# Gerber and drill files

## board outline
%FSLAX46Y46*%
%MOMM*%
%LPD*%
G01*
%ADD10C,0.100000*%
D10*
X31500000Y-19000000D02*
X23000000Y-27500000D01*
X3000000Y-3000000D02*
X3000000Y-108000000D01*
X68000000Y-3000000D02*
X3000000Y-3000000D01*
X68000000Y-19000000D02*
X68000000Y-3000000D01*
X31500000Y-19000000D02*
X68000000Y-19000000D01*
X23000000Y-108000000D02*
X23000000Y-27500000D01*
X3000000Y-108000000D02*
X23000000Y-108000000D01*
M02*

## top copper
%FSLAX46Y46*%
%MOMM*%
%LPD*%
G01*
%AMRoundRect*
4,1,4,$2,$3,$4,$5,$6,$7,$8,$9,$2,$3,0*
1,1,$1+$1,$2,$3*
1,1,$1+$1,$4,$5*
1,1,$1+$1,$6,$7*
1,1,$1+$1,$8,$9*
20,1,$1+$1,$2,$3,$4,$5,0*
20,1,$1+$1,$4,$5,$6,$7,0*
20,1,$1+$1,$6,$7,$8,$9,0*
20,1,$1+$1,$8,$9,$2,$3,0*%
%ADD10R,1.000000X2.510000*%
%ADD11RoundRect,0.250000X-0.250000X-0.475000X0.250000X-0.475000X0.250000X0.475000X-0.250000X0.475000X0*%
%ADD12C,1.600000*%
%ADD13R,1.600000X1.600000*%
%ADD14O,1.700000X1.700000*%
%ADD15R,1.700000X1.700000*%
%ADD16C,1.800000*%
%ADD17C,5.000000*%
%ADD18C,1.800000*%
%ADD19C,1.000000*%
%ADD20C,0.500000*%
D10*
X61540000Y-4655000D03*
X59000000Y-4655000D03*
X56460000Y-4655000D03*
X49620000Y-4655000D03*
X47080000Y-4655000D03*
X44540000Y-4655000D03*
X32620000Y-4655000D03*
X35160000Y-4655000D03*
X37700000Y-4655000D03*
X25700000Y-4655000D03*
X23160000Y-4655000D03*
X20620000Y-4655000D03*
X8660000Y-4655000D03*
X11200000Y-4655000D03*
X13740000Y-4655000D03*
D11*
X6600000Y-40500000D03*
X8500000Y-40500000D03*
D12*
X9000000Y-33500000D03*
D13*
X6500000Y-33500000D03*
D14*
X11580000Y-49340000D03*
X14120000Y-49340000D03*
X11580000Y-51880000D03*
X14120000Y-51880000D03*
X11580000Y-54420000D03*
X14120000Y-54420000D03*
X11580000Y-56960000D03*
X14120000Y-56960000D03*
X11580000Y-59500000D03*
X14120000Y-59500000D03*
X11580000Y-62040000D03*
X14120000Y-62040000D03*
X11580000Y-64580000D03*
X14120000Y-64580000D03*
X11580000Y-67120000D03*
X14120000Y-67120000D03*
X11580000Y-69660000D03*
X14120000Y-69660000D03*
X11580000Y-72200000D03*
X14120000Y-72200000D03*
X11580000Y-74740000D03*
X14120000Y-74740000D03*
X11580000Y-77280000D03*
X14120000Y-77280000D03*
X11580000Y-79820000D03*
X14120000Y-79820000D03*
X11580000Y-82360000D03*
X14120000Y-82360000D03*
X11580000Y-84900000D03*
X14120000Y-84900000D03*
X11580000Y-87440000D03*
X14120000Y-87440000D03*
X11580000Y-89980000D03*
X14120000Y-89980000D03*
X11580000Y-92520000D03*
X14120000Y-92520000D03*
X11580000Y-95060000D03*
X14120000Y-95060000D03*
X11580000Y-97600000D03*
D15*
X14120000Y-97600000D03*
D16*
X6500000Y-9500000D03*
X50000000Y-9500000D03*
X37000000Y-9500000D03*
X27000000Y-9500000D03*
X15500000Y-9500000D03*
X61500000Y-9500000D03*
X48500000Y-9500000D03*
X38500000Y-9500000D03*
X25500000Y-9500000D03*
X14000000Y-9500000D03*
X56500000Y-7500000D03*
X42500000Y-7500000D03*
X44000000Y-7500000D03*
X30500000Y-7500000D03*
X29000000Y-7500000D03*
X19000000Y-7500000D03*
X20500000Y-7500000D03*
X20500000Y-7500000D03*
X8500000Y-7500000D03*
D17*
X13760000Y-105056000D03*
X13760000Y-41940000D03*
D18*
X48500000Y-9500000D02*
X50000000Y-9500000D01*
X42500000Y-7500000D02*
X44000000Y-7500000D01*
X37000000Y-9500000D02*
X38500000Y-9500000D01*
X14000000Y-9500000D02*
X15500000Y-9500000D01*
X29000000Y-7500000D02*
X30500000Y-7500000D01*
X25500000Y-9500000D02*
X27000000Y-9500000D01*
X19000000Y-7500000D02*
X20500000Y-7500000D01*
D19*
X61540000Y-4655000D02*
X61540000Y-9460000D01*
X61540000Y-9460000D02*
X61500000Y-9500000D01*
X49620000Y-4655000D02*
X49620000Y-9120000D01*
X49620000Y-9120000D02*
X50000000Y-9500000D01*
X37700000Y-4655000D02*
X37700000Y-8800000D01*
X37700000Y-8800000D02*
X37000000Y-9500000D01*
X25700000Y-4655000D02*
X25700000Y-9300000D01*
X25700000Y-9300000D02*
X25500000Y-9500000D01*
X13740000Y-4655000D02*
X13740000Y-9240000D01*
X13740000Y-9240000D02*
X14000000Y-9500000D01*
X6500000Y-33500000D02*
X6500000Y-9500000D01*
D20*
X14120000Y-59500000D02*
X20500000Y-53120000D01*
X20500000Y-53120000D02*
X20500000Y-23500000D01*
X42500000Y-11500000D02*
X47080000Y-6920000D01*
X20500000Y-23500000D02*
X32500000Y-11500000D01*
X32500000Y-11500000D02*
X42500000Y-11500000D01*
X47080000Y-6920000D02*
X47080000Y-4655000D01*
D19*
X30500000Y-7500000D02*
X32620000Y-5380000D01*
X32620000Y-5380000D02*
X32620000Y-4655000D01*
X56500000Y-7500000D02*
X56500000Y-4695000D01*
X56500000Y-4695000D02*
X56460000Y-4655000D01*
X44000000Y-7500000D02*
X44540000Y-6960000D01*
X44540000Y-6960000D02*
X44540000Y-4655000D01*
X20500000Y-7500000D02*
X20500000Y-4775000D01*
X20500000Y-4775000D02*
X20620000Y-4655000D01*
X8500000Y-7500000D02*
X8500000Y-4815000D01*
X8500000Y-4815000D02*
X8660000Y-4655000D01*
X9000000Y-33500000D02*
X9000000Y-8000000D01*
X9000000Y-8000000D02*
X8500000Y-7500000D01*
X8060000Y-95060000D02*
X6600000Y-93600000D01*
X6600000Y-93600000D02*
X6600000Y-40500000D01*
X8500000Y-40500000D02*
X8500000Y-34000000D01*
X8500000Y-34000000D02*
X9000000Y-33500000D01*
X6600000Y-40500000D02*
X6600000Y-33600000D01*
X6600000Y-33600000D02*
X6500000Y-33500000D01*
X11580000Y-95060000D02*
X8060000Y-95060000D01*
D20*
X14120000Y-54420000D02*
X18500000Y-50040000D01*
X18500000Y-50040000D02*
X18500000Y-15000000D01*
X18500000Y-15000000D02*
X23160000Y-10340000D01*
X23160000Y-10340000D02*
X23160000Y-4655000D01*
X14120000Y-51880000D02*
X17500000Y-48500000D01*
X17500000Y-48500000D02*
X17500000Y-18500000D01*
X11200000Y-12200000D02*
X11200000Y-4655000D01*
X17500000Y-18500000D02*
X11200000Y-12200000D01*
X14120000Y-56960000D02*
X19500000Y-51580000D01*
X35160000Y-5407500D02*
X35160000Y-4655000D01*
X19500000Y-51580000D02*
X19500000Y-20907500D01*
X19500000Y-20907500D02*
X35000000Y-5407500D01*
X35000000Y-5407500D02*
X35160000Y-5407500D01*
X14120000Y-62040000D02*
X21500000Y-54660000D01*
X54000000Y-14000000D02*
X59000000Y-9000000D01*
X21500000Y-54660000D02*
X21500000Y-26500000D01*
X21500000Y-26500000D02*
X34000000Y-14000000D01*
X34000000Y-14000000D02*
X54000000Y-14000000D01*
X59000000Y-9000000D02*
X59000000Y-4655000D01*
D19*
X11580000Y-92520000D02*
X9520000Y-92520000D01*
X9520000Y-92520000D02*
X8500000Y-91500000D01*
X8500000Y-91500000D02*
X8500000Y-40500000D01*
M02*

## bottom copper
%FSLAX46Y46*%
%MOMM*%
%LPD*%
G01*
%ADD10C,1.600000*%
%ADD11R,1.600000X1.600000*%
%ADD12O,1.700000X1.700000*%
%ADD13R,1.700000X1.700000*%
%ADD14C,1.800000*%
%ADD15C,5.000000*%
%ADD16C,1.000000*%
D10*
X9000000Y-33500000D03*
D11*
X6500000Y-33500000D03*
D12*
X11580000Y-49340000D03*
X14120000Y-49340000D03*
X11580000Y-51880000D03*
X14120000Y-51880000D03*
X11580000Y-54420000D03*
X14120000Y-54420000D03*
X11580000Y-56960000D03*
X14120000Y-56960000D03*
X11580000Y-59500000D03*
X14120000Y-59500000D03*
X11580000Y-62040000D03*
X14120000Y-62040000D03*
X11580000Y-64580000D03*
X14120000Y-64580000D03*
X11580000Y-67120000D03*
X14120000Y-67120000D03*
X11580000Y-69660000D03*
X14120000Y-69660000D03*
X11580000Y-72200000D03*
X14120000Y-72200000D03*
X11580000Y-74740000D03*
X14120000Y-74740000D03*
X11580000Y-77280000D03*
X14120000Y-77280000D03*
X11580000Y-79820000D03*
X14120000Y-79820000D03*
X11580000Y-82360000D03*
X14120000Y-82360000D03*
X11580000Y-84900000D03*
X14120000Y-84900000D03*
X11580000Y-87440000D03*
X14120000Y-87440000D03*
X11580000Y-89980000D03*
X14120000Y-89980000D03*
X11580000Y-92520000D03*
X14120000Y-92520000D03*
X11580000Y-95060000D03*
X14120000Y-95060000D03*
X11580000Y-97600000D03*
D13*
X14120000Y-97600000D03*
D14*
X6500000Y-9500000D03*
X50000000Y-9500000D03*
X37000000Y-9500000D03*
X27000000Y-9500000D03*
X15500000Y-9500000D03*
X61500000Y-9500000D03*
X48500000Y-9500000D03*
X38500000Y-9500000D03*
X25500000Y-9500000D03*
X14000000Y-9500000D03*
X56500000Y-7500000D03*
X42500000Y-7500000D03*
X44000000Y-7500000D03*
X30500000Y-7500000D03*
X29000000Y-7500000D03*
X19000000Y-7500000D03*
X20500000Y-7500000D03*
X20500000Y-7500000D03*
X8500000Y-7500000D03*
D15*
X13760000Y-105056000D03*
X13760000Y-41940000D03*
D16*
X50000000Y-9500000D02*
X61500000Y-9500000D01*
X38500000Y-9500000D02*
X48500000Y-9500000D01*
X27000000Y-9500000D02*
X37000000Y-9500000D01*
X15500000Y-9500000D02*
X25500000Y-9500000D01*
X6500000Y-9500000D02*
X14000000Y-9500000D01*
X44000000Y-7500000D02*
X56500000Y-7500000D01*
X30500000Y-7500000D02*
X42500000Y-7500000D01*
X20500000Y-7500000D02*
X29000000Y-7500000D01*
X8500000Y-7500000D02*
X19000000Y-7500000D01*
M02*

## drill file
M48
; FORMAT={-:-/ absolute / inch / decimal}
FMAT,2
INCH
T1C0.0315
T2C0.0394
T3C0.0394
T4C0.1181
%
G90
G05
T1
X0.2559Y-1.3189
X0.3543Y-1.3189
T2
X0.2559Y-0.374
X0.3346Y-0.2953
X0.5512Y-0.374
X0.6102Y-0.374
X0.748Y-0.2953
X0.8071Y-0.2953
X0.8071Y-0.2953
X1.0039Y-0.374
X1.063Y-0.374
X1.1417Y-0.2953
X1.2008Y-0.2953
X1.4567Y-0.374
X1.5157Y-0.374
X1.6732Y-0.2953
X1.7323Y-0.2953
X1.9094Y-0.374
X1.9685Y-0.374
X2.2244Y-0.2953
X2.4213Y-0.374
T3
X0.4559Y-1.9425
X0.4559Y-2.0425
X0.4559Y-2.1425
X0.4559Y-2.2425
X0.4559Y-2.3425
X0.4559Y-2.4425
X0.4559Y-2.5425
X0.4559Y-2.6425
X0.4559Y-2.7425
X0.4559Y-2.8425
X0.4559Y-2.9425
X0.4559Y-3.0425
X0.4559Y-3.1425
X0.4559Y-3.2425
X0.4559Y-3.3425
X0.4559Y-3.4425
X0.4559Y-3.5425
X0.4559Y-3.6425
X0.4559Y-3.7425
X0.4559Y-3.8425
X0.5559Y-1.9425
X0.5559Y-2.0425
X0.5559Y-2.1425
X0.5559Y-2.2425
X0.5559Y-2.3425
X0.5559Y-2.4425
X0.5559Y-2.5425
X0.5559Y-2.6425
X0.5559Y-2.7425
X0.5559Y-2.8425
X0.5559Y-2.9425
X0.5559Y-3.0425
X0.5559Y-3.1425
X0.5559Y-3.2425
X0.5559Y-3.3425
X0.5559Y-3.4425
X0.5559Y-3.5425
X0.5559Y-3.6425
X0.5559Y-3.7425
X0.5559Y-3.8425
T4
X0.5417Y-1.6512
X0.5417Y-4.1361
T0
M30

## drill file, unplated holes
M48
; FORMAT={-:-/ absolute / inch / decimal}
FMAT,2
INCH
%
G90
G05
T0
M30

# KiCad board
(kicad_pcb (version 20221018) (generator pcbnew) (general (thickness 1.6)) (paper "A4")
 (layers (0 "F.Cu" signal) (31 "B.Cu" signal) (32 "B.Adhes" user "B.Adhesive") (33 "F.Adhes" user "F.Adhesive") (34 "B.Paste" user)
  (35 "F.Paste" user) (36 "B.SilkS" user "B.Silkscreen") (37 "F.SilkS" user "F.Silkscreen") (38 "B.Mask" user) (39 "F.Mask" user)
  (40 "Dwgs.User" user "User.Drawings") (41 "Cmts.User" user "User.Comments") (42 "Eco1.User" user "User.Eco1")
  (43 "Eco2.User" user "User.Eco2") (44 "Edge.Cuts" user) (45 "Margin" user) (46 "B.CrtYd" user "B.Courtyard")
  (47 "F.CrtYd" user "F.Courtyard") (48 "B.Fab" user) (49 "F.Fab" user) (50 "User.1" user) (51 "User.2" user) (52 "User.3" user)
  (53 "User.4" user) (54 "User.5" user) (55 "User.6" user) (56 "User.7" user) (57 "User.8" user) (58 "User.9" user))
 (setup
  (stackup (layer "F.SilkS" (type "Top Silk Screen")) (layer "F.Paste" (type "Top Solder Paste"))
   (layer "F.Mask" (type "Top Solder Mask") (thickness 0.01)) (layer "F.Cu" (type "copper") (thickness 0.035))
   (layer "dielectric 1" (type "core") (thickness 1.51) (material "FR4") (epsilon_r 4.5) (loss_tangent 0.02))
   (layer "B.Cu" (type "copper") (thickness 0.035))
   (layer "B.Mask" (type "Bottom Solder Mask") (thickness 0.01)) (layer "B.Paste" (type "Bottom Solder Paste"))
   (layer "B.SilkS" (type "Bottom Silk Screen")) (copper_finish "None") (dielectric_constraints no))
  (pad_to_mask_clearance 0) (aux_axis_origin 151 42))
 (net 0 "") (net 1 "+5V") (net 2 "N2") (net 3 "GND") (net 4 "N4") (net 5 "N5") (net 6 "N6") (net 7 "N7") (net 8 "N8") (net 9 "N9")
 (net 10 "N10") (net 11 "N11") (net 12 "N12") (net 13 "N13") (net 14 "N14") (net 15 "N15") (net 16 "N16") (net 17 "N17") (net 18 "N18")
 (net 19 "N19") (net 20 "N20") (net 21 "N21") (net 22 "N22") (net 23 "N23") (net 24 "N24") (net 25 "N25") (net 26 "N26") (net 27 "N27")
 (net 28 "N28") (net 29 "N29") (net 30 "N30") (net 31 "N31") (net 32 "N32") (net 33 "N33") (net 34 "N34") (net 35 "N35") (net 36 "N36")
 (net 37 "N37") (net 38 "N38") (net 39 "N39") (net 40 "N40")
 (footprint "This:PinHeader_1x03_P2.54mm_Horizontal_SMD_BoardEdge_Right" (layer "F.Cu") (at 174.16 45 -90)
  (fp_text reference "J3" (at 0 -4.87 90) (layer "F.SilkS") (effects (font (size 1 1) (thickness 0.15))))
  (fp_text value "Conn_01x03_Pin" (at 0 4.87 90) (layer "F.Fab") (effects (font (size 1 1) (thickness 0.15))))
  (pad "1" smd rect (at 1.655 -2.54 270) (size 2.51 1) (layers "F.Cu" "F.Paste" "F.Mask") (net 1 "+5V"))
  (pad "2" smd rect (at 1.655 0 270) (size 2.51 1) (layers "F.Cu" "F.Paste" "F.Mask") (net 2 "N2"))
  (pad "3" smd rect (at 1.655 2.54 270) (size 2.51 1) (layers "F.Cu" "F.Paste" "F.Mask") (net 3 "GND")))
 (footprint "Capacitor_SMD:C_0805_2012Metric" (layer "F.Cu") (at 158.55 82.5)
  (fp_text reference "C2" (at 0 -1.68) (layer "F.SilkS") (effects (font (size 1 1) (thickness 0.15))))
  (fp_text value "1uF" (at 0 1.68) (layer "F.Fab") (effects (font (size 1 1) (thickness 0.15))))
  (pad "1" smd roundrect (at -0.95 0) (size 1 1.45) (layers "F.Cu" "F.Paste" "F.Mask") (roundrect_rratio 0.25) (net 1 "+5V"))
  (pad "2" smd roundrect (at 0.95 0) (size 1 1.45) (layers "F.Cu" "F.Paste" "F.Mask") (roundrect_rratio 0.25) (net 3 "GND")))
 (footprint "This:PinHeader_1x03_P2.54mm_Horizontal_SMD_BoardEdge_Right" (layer "F.Cu") (at 162.2 45 -90)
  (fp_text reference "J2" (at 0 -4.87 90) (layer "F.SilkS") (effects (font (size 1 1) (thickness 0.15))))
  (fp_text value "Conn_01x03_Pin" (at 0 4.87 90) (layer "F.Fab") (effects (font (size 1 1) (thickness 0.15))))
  (pad "1" smd rect (at 1.655 -2.54 270) (size 2.51 1) (layers "F.Cu" "F.Paste" "F.Mask") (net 1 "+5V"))
  (pad "2" smd rect (at 1.655 0 270) (size 2.51 1) (layers "F.Cu" "F.Paste" "F.Mask") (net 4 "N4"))
  (pad "3" smd rect (at 1.655 2.54 270) (size 2.51 1) (layers "F.Cu" "F.Paste" "F.Mask") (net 3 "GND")))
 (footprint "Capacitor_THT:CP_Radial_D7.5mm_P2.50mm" (layer "F.Cu") (at 157.5 75.5)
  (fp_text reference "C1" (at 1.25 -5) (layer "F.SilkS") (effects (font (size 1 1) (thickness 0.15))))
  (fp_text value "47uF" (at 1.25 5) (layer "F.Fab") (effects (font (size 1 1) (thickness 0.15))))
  (pad "1" thru_hole rect (at 0 0) (size 1.6 1.6) (drill 0.8) (layers "*.Cu" "*.Mask") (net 1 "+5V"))
  (pad "2" thru_hole circle (at 2.5 0) (size 1.6 1.6) (drill 0.8) (layers "*.Cu" "*.Mask") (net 3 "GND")))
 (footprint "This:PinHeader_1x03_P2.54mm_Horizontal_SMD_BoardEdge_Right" (layer "F.Cu") (at 210 45 -90)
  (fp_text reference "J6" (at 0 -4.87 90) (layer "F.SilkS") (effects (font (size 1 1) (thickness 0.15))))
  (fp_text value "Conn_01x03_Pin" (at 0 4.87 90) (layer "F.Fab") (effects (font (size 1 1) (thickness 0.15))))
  (pad "1" smd rect (at 1.655 -2.54 270) (size 2.51 1) (layers "F.Cu" "F.Paste" "F.Mask") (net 1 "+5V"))
  (pad "2" smd rect (at 1.655 0 270) (size 2.51 1) (layers "F.Cu" "F.Paste" "F.Mask") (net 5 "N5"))
  (pad "3" smd rect (at 1.655 2.54 270) (size 2.51 1) (layers "F.Cu" "F.Paste" "F.Mask") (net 3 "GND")))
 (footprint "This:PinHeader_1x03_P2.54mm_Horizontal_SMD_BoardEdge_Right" (layer "F.Cu") (at 186.16 45 -90)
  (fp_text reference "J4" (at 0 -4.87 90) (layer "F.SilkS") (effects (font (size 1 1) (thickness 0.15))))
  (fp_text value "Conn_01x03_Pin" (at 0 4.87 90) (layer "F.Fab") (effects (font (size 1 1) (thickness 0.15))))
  (pad "1" smd rect (at 1.655 -2.54 270) (size 2.51 1) (layers "F.Cu" "F.Paste" "F.Mask") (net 1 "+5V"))
  (pad "2" smd rect (at 1.655 0 270) (size 2.51 1) (layers "F.Cu" "F.Paste" "F.Mask") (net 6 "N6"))
  (pad "3" smd rect (at 1.655 2.54 270) (size 2.51 1) (layers "F.Cu" "F.Paste" "F.Mask") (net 3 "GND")))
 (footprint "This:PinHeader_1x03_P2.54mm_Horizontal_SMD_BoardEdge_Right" (layer "F.Cu") (at 198.08 45 -90)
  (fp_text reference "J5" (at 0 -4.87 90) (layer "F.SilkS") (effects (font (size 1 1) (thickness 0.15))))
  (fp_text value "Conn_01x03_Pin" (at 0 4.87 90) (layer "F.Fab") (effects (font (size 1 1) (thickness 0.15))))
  (pad "1" smd rect (at 1.655 -2.54 270) (size 2.51 1) (layers "F.Cu" "F.Paste" "F.Mask") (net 1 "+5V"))
  (pad "2" smd rect (at 1.655 0 270) (size 2.51 1) (layers "F.Cu" "F.Paste" "F.Mask") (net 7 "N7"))
  (pad "3" smd rect (at 1.655 2.54 270) (size 2.51 1) (layers "F.Cu" "F.Paste" "F.Mask") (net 3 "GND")))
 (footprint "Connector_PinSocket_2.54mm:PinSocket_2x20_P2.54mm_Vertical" (layer "B.Cu") (at 165.12 139.6)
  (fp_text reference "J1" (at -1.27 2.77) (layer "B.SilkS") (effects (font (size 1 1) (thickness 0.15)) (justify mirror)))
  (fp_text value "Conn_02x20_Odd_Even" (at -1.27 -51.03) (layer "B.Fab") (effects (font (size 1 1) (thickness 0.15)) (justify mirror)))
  (pad "1" thru_hole rect (at 0 0) (size 1.7 1.7) (drill 1) (layers "*.Cu" "*.Mask") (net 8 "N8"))
  (pad "2" thru_hole oval (at -2.54 0) (size 1.7 1.7) (drill 1) (layers "*.Cu" "*.Mask") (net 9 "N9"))
  (pad "3" thru_hole oval (at 0 -2.54) (size 1.7 1.7) (drill 1) (layers "*.Cu" "*.Mask") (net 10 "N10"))
  (pad "4" thru_hole oval (at -2.54 -2.54) (size 1.7 1.7) (drill 1) (layers "*.Cu" "*.Mask") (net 1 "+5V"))
  (pad "5" thru_hole oval (at 0 -5.08) (size 1.7 1.7) (drill 1) (layers "*.Cu" "*.Mask") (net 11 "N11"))
  (pad "6" thru_hole oval (at -2.54 -5.08) (size 1.7 1.7) (drill 1) (layers "*.Cu" "*.Mask") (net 3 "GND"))
  (pad "7" thru_hole oval (at 0 -7.62) (size 1.7 1.7) (drill 1) (layers "*.Cu" "*.Mask") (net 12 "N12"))
  (pad "8" thru_hole oval (at -2.54 -7.62) (size 1.7 1.7) (drill 1) (layers "*.Cu" "*.Mask") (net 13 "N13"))
  (pad "9" thru_hole oval (at 0 -10.16) (size 1.7 1.7) (drill 1) (layers "*.Cu" "*.Mask") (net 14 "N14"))
  (pad "10" thru_hole oval (at -2.54 -10.16) (size 1.7 1.7) (drill 1) (layers "*.Cu" "*.Mask") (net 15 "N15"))
  (pad "11" thru_hole oval (at 0 -12.7) (size 1.7 1.7) (drill 1) (layers "*.Cu" "*.Mask") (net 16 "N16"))
  (pad "12" thru_hole oval (at -2.54 -12.7) (size 1.7 1.7) (drill 1) (layers "*.Cu" "*.Mask") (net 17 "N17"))
  (pad "13" thru_hole oval (at 0 -15.24) (size 1.7 1.7) (drill 1) (layers "*.Cu" "*.Mask") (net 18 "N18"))
  (pad "14" thru_hole oval (at -2.54 -15.24) (size 1.7 1.7) (drill 1) (layers "*.Cu" "*.Mask") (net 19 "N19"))
  (pad "15" thru_hole oval (at 0 -17.78) (size 1.7 1.7) (drill 1) (layers "*.Cu" "*.Mask") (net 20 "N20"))
  (pad "16" thru_hole oval (at -2.54 -17.78) (size 1.7 1.7) (drill 1) (layers "*.Cu" "*.Mask") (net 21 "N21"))
  (pad "17" thru_hole oval (at 0 -20.32) (size 1.7 1.7) (drill 1) (layers "*.Cu" "*.Mask") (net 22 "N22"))
  (pad "18" thru_hole oval (at -2.54 -20.32) (size 1.7 1.7) (drill 1) (layers "*.Cu" "*.Mask") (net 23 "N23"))
  (pad "19" thru_hole oval (at 0 -22.86) (size 1.7 1.7) (drill 1) (layers "*.Cu" "*.Mask") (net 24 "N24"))
  (pad "20" thru_hole oval (at -2.54 -22.86) (size 1.7 1.7) (drill 1) (layers "*.Cu" "*.Mask") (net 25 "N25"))
  (pad "21" thru_hole oval (at 0 -25.4) (size 1.7 1.7) (drill 1) (layers "*.Cu" "*.Mask") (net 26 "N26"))
  (pad "22" thru_hole oval (at -2.54 -25.4) (size 1.7 1.7) (drill 1) (layers "*.Cu" "*.Mask") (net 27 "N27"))
  (pad "23" thru_hole oval (at 0 -27.94) (size 1.7 1.7) (drill 1) (layers "*.Cu" "*.Mask") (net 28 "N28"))
  (pad "24" thru_hole oval (at -2.54 -27.94) (size 1.7 1.7) (drill 1) (layers "*.Cu" "*.Mask") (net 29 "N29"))
  (pad "25" thru_hole oval (at 0 -30.48) (size 1.7 1.7) (drill 1) (layers "*.Cu" "*.Mask") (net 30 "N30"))
  (pad "26" thru_hole oval (at -2.54 -30.48) (size 1.7 1.7) (drill 1) (layers "*.Cu" "*.Mask") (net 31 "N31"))
  (pad "27" thru_hole oval (at 0 -33.02) (size 1.7 1.7) (drill 1) (layers "*.Cu" "*.Mask") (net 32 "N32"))
  (pad "28" thru_hole oval (at -2.54 -33.02) (size 1.7 1.7) (drill 1) (layers "*.Cu" "*.Mask") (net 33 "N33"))
  (pad "29" thru_hole oval (at 0 -35.56) (size 1.7 1.7) (drill 1) (layers "*.Cu" "*.Mask") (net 5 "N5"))
  (pad "30" thru_hole oval (at -2.54 -35.56) (size 1.7 1.7) (drill 1) (layers "*.Cu" "*.Mask") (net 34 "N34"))
  (pad "31" thru_hole oval (at 0 -38.1) (size 1.7 1.7) (drill 1) (layers "*.Cu" "*.Mask") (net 7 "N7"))
  (pad "32" thru_hole oval (at -2.54 -38.1) (size 1.7 1.7) (drill 1) (layers "*.Cu" "*.Mask") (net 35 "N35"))
  (pad "33" thru_hole oval (at 0 -40.64) (size 1.7 1.7) (drill 1) (layers "*.Cu" "*.Mask") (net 6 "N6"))
  (pad "34" thru_hole oval (at -2.54 -40.64) (size 1.7 1.7) (drill 1) (layers "*.Cu" "*.Mask") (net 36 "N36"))
  (pad "35" thru_hole oval (at 0 -43.18) (size 1.7 1.7) (drill 1) (layers "*.Cu" "*.Mask") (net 2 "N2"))
  (pad "36" thru_hole oval (at -2.54 -43.18) (size 1.7 1.7) (drill 1) (layers "*.Cu" "*.Mask") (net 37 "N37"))
  (pad "37" thru_hole oval (at 0 -45.72) (size 1.7 1.7) (drill 1) (layers "*.Cu" "*.Mask") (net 4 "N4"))
  (pad "38" thru_hole oval (at -2.54 -45.72) (size 1.7 1.7) (drill 1) (layers "*.Cu" "*.Mask") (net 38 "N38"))
  (pad "39" thru_hole oval (at 0 -48.26) (size 1.7 1.7) (drill 1) (layers "*.Cu" "*.Mask") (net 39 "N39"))
  (pad "40" thru_hole oval (at -2.54 -48.26) (size 1.7 1.7) (drill 1) (layers "*.Cu" "*.Mask") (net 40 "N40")))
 (gr_line (start 154 45) (end 154 150) (stroke (width 0.1) (type default)) (layer "Edge.Cuts"))
 (gr_line (start 219 45) (end 154 45) (stroke (width 0.1) (type default)) (layer "Edge.Cuts"))
 (gr_line (start 219 61) (end 219 45) (stroke (width 0.1) (type default)) (layer "Edge.Cuts"))
 (gr_line (start 182.5 61) (end 174 69.5) (stroke (width 0.1) (type default)) (layer "Edge.Cuts"))
 (gr_line (start 182.5 61) (end 219 61) (stroke (width 0.1) (type default)) (layer "Edge.Cuts"))
 (gr_line (start 174 150) (end 174 69.5) (stroke (width 0.1) (type default)) (layer "Edge.Cuts"))
 (gr_line (start 154 150) (end 174 150) (stroke (width 0.1) (type default)) (layer "Edge.Cuts"))
 (via (at 164.76 147.056) (size 5) (drill 3) (layers "F.Cu" "B.Cu") (free) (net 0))
 (via (at 164.76 83.94) (size 5) (drill 3) (layers "F.Cu" "B.Cu") (free) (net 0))
 (segment (start 195 49.5) (end 195.54 48.96) (width 1) (layer "F.Cu") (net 3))
 (segment (start 159.5 133.5) (end 159.5 82.5) (width 1) (layer "F.Cu") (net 3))
 (segment (start 162.58 134.52) (end 160.52 134.52) (width 1) (layer "F.Cu") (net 3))
 (segment (start 207.5 49.5) (end 207.5 46.695) (width 1) (layer "F.Cu") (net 3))
 (segment (start 171.5 49.5) (end 171.5 46.775) (width 1) (layer "F.Cu") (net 3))
 (segment (start 170 49.5) (end 171.5 49.5) (width 1.8) (layer "F.Cu") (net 3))
 (segment (start 183.62 47.38) (end 183.62 46.655) (width 1) (layer "F.Cu") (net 3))
 (segment (start 159.5 49.5) (end 159.5 46.815) (width 1) (layer "F.Cu") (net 3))
 (segment (start 160.52 134.52) (end 159.5 133.5) (width 1) (layer "F.Cu") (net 3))
 (segment (start 195.54 48.96) (end 195.54 46.655) (width 1) (layer "F.Cu") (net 3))
 (segment (start 160 50) (end 159.5 49.5) (width 1) (layer "F.Cu") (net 3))
 (segment (start 207.5 46.695) (end 207.46 46.655) (width 1) (layer "F.Cu") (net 3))
 (segment (start 160 75.5) (end 160 50) (width 1) (layer "F.Cu") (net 3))
 (segment (start 159.5 46.815) (end 159.66 46.655) (width 1) (layer "F.Cu") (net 3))
 (segment (start 193.5 49.5) (end 195 49.5) (width 1.8) (layer "F.Cu") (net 3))
 (segment (start 159.5 76) (end 160 75.5) (width 1) (layer "F.Cu") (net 3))
 (segment (start 180 49.5) (end 181.5 49.5) (width 1.8) (layer "F.Cu") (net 3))
 (segment (start 159.5 82.5) (end 159.5 76) (width 1) (layer "F.Cu") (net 3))
 (segment (start 171.5 46.775) (end 171.62 46.655) (width 1) (layer "F.Cu") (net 3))
 (segment (start 181.5 49.5) (end 183.62 47.38) (width 1) (layer "F.Cu") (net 3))
 (via (at 195 49.5) (size 1.8) (drill 1) (layers "F.Cu" "B.Cu") (free) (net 3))
 (via (at 181.5 49.5) (size 1.8) (drill 1) (layers "F.Cu" "B.Cu") (free) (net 3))
 (via (at 171.5 49.5) (size 1.8) (drill 1) (layers "F.Cu" "B.Cu") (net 3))
 (via (at 207.5 49.5) (size 1.8) (drill 1) (layers "F.Cu" "B.Cu") (free) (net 3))
 (via (at 170 49.5) (size 1.8) (drill 1) (layers "F.Cu" "B.Cu") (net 3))
 (via (at 159.5 49.5) (size 1.8) (drill 1) (layers "F.Cu" "B.Cu") (free) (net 3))
 (via (at 193.5 49.5) (size 1.8) (drill 1) (layers "F.Cu" "B.Cu") (free) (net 3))
 (via (at 171.5 49.5) (size 1.8) (drill 1) (layers "F.Cu" "B.Cu") (free) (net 3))
 (via (at 180 49.5) (size 1.8) (drill 1) (layers "F.Cu" "B.Cu") (free) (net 3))
 (segment (start 171.5 49.5) (end 180 49.5) (width 1) (layer "B.Cu") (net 3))
 (segment (start 181.5 49.5) (end 193.5 49.5) (width 1) (layer "B.Cu") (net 3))
 (segment (start 159.5 49.5) (end 170 49.5) (width 1) (layer "B.Cu") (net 3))
 (segment (start 195 49.5) (end 207.5 49.5) (width 1) (layer "B.Cu") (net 3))
 (segment (start 188 51.5) (end 189.5 51.5) (width 1.8) (layer "F.Cu") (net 1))
 (segment (start 199.5 51.5) (end 201 51.5) (width 1.8) (layer "F.Cu") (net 1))
 (segment (start 188.7 50.8) (end 188 51.5) (width 1) (layer "F.Cu") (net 1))
 (segment (start 157.6 135.6) (end 157.6 82.5) (width 1) (layer "F.Cu") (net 1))
 (segment (start 157.5 75.5) (end 157.5 51.5) (width 1) (layer "F.Cu") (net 1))
 (segment (start 176.7 51.3) (end 176.5 51.5) (width 1) (layer "F.Cu") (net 1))
 (segment (start 200.62 51.12) (end 201 51.5) (width 1) (layer "F.Cu") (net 1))
 (segment (start 212.54 51.46) (end 212.5 51.5) (width 1) (layer "F.Cu") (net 1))
 (segment (start 176.7 46.655) (end 176.7 51.3) (width 1) (layer "F.Cu") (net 1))
 (segment (start 165 51.5) (end 166.5 51.5) (width 1.8) (layer "F.Cu") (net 1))
 (segment (start 162.58 137.06) (end 159.06 137.06) (width 1) (layer "F.Cu") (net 1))
 (segment (start 157.6 75.6) (end 157.5 75.5) (width 1) (layer "F.Cu") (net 1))
 (segment (start 176.5 51.5) (end 178 51.5) (width 1.8) (layer "F.Cu") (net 1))
 (segment (start 164.74 46.655) (end 164.74 51.24) (width 1) (layer "F.Cu") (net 1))
 (segment (start 157.6 82.5) (end 157.6 75.6) (width 1) (layer "F.Cu") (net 1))
 (segment (start 188.7 46.655) (end 188.7 50.8) (width 1) (layer "F.Cu") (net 1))
 (segment (start 159.06 137.06) (end 157.6 135.6) (width 1) (layer "F.Cu") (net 1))
 (segment (start 164.74 51.24) (end 165 51.5) (width 1) (layer "F.Cu") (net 1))
 (segment (start 212.54 46.655) (end 212.54 51.46) (width 1) (layer "F.Cu") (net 1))
 (segment (start 200.62 46.655) (end 200.62 51.12) (width 1) (layer "F.Cu") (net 1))
 (via (at 212.5 51.5) (size 1.8) (drill 1) (layers "F.Cu" "B.Cu") (free) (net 1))
 (via (at 176.5 51.5) (size 1.8) (drill 1) (layers "F.Cu" "B.Cu") (free) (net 1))
 (via (at 188 51.5) (size 1.8) (drill 1) (layers "F.Cu" "B.Cu") (free) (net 1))
 (via (at 165 51.5) (size 1.8) (drill 1) (layers "F.Cu" "B.Cu") (free) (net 1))
 (via (at 199.5 51.5) (size 1.8) (drill 1) (layers "F.Cu" "B.Cu") (free) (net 1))
 (via (at 201 51.5) (size 1.8) (drill 1) (layers "F.Cu" "B.Cu") (free) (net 1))
 (via (at 189.5 51.5) (size 1.8) (drill 1) (layers "F.Cu" "B.Cu") (free) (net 1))
 (via (at 157.5 51.5) (size 1.8) (drill 1) (layers "F.Cu" "B.Cu") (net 1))
 (via (at 166.5 51.5) (size 1.8) (drill 1) (layers "F.Cu" "B.Cu") (free) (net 1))
 (via (at 178 51.5) (size 1.8) (drill 1) (layers "F.Cu" "B.Cu") (free) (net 1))
 (segment (start 201 51.5) (end 212.5 51.5) (width 1) (layer "B.Cu") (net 1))
 (segment (start 178 51.5) (end 188 51.5) (width 1) (layer "B.Cu") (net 1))
 (segment (start 189.5 51.5) (end 199.5 51.5) (width 1) (layer "B.Cu") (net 1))
 (segment (start 166.5 51.5) (end 176.5 51.5) (width 1) (layer "B.Cu") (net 1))
 (segment (start 157.5 51.5) (end 165 51.5) (width 1) (layer "B.Cu") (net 1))
 (segment (start 172.5 68.5) (end 185 56) (width 0.5) (layer "F.Cu") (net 5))
 (segment (start 172.5 96.66) (end 172.5 68.5) (width 0.5) (layer "F.Cu") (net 5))
 (segment (start 205 56) (end 210 51) (width 0.5) (layer "F.Cu") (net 5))
 (segment (start 185 56) (end 205 56) (width 0.5) (layer "F.Cu") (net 5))
 (segment (start 165.12 104.04) (end 172.5 96.66) (width 0.5) (layer "F.Cu") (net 5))
 (segment (start 210 51) (end 210 46.655) (width 0.5) (layer "F.Cu") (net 5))
 (segment (start 198.08 48.92) (end 198.08 46.655) (width 0.5) (layer "F.Cu") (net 7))
 (segment (start 193.5 53.5) (end 198.08 48.92) (width 0.5) (layer "F.Cu") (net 7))
 (segment (start 165.12 101.5) (end 171.5 95.12) (width 0.5) (layer "F.Cu") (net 7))
 (segment (start 171.5 65.5) (end 183.5 53.5) (width 0.5) (layer "F.Cu") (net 7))
 (segment (start 183.5 53.5) (end 193.5 53.5) (width 0.5) (layer "F.Cu") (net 7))
 (segment (start 171.5 95.12) (end 171.5 65.5) (width 0.5) (layer "F.Cu") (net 7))
 (segment (start 170.5 62.9075) (end 186 47.4075) (width 0.5) (layer "F.Cu") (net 6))
 (segment (start 170.5 93.58) (end 170.5 62.9075) (width 0.5) (layer "F.Cu") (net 6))
 (segment (start 186 47.4075) (end 186.16 47.4075) (width 0.5) (layer "F.Cu") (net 6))
 (segment (start 186.16 47.4075) (end 186.16 46.655) (width 0.5) (layer "F.Cu") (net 6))
 (segment (start 165.12 98.96) (end 170.5 93.58) (width 0.5) (layer "F.Cu") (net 6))
 (segment (start 169.5 57) (end 174.16 52.34) (width 0.5) (layer "F.Cu") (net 2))
 (segment (start 169.5 92.04) (end 169.5 57) (width 0.5) (layer "F.Cu") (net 2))
 (segment (start 165.12 96.42) (end 169.5 92.04) (width 0.5) (layer "F.Cu") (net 2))
 (segment (start 174.16 52.34) (end 174.16 46.655) (width 0.5) (layer "F.Cu") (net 2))
 (segment (start 168.5 60.5) (end 162.2 54.2) (width 0.5) (layer "F.Cu") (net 4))
 (segment (start 162.2 54.2) (end 162.2 46.655) (width 0.5) (layer "F.Cu") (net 4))
 (segment (start 165.12 93.88) (end 168.5 90.5) (width 0.5) (layer "F.Cu") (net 4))
 (segment (start 168.5 90.5) (end 168.5 60.5) (width 0.5) (layer "F.Cu") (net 4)))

